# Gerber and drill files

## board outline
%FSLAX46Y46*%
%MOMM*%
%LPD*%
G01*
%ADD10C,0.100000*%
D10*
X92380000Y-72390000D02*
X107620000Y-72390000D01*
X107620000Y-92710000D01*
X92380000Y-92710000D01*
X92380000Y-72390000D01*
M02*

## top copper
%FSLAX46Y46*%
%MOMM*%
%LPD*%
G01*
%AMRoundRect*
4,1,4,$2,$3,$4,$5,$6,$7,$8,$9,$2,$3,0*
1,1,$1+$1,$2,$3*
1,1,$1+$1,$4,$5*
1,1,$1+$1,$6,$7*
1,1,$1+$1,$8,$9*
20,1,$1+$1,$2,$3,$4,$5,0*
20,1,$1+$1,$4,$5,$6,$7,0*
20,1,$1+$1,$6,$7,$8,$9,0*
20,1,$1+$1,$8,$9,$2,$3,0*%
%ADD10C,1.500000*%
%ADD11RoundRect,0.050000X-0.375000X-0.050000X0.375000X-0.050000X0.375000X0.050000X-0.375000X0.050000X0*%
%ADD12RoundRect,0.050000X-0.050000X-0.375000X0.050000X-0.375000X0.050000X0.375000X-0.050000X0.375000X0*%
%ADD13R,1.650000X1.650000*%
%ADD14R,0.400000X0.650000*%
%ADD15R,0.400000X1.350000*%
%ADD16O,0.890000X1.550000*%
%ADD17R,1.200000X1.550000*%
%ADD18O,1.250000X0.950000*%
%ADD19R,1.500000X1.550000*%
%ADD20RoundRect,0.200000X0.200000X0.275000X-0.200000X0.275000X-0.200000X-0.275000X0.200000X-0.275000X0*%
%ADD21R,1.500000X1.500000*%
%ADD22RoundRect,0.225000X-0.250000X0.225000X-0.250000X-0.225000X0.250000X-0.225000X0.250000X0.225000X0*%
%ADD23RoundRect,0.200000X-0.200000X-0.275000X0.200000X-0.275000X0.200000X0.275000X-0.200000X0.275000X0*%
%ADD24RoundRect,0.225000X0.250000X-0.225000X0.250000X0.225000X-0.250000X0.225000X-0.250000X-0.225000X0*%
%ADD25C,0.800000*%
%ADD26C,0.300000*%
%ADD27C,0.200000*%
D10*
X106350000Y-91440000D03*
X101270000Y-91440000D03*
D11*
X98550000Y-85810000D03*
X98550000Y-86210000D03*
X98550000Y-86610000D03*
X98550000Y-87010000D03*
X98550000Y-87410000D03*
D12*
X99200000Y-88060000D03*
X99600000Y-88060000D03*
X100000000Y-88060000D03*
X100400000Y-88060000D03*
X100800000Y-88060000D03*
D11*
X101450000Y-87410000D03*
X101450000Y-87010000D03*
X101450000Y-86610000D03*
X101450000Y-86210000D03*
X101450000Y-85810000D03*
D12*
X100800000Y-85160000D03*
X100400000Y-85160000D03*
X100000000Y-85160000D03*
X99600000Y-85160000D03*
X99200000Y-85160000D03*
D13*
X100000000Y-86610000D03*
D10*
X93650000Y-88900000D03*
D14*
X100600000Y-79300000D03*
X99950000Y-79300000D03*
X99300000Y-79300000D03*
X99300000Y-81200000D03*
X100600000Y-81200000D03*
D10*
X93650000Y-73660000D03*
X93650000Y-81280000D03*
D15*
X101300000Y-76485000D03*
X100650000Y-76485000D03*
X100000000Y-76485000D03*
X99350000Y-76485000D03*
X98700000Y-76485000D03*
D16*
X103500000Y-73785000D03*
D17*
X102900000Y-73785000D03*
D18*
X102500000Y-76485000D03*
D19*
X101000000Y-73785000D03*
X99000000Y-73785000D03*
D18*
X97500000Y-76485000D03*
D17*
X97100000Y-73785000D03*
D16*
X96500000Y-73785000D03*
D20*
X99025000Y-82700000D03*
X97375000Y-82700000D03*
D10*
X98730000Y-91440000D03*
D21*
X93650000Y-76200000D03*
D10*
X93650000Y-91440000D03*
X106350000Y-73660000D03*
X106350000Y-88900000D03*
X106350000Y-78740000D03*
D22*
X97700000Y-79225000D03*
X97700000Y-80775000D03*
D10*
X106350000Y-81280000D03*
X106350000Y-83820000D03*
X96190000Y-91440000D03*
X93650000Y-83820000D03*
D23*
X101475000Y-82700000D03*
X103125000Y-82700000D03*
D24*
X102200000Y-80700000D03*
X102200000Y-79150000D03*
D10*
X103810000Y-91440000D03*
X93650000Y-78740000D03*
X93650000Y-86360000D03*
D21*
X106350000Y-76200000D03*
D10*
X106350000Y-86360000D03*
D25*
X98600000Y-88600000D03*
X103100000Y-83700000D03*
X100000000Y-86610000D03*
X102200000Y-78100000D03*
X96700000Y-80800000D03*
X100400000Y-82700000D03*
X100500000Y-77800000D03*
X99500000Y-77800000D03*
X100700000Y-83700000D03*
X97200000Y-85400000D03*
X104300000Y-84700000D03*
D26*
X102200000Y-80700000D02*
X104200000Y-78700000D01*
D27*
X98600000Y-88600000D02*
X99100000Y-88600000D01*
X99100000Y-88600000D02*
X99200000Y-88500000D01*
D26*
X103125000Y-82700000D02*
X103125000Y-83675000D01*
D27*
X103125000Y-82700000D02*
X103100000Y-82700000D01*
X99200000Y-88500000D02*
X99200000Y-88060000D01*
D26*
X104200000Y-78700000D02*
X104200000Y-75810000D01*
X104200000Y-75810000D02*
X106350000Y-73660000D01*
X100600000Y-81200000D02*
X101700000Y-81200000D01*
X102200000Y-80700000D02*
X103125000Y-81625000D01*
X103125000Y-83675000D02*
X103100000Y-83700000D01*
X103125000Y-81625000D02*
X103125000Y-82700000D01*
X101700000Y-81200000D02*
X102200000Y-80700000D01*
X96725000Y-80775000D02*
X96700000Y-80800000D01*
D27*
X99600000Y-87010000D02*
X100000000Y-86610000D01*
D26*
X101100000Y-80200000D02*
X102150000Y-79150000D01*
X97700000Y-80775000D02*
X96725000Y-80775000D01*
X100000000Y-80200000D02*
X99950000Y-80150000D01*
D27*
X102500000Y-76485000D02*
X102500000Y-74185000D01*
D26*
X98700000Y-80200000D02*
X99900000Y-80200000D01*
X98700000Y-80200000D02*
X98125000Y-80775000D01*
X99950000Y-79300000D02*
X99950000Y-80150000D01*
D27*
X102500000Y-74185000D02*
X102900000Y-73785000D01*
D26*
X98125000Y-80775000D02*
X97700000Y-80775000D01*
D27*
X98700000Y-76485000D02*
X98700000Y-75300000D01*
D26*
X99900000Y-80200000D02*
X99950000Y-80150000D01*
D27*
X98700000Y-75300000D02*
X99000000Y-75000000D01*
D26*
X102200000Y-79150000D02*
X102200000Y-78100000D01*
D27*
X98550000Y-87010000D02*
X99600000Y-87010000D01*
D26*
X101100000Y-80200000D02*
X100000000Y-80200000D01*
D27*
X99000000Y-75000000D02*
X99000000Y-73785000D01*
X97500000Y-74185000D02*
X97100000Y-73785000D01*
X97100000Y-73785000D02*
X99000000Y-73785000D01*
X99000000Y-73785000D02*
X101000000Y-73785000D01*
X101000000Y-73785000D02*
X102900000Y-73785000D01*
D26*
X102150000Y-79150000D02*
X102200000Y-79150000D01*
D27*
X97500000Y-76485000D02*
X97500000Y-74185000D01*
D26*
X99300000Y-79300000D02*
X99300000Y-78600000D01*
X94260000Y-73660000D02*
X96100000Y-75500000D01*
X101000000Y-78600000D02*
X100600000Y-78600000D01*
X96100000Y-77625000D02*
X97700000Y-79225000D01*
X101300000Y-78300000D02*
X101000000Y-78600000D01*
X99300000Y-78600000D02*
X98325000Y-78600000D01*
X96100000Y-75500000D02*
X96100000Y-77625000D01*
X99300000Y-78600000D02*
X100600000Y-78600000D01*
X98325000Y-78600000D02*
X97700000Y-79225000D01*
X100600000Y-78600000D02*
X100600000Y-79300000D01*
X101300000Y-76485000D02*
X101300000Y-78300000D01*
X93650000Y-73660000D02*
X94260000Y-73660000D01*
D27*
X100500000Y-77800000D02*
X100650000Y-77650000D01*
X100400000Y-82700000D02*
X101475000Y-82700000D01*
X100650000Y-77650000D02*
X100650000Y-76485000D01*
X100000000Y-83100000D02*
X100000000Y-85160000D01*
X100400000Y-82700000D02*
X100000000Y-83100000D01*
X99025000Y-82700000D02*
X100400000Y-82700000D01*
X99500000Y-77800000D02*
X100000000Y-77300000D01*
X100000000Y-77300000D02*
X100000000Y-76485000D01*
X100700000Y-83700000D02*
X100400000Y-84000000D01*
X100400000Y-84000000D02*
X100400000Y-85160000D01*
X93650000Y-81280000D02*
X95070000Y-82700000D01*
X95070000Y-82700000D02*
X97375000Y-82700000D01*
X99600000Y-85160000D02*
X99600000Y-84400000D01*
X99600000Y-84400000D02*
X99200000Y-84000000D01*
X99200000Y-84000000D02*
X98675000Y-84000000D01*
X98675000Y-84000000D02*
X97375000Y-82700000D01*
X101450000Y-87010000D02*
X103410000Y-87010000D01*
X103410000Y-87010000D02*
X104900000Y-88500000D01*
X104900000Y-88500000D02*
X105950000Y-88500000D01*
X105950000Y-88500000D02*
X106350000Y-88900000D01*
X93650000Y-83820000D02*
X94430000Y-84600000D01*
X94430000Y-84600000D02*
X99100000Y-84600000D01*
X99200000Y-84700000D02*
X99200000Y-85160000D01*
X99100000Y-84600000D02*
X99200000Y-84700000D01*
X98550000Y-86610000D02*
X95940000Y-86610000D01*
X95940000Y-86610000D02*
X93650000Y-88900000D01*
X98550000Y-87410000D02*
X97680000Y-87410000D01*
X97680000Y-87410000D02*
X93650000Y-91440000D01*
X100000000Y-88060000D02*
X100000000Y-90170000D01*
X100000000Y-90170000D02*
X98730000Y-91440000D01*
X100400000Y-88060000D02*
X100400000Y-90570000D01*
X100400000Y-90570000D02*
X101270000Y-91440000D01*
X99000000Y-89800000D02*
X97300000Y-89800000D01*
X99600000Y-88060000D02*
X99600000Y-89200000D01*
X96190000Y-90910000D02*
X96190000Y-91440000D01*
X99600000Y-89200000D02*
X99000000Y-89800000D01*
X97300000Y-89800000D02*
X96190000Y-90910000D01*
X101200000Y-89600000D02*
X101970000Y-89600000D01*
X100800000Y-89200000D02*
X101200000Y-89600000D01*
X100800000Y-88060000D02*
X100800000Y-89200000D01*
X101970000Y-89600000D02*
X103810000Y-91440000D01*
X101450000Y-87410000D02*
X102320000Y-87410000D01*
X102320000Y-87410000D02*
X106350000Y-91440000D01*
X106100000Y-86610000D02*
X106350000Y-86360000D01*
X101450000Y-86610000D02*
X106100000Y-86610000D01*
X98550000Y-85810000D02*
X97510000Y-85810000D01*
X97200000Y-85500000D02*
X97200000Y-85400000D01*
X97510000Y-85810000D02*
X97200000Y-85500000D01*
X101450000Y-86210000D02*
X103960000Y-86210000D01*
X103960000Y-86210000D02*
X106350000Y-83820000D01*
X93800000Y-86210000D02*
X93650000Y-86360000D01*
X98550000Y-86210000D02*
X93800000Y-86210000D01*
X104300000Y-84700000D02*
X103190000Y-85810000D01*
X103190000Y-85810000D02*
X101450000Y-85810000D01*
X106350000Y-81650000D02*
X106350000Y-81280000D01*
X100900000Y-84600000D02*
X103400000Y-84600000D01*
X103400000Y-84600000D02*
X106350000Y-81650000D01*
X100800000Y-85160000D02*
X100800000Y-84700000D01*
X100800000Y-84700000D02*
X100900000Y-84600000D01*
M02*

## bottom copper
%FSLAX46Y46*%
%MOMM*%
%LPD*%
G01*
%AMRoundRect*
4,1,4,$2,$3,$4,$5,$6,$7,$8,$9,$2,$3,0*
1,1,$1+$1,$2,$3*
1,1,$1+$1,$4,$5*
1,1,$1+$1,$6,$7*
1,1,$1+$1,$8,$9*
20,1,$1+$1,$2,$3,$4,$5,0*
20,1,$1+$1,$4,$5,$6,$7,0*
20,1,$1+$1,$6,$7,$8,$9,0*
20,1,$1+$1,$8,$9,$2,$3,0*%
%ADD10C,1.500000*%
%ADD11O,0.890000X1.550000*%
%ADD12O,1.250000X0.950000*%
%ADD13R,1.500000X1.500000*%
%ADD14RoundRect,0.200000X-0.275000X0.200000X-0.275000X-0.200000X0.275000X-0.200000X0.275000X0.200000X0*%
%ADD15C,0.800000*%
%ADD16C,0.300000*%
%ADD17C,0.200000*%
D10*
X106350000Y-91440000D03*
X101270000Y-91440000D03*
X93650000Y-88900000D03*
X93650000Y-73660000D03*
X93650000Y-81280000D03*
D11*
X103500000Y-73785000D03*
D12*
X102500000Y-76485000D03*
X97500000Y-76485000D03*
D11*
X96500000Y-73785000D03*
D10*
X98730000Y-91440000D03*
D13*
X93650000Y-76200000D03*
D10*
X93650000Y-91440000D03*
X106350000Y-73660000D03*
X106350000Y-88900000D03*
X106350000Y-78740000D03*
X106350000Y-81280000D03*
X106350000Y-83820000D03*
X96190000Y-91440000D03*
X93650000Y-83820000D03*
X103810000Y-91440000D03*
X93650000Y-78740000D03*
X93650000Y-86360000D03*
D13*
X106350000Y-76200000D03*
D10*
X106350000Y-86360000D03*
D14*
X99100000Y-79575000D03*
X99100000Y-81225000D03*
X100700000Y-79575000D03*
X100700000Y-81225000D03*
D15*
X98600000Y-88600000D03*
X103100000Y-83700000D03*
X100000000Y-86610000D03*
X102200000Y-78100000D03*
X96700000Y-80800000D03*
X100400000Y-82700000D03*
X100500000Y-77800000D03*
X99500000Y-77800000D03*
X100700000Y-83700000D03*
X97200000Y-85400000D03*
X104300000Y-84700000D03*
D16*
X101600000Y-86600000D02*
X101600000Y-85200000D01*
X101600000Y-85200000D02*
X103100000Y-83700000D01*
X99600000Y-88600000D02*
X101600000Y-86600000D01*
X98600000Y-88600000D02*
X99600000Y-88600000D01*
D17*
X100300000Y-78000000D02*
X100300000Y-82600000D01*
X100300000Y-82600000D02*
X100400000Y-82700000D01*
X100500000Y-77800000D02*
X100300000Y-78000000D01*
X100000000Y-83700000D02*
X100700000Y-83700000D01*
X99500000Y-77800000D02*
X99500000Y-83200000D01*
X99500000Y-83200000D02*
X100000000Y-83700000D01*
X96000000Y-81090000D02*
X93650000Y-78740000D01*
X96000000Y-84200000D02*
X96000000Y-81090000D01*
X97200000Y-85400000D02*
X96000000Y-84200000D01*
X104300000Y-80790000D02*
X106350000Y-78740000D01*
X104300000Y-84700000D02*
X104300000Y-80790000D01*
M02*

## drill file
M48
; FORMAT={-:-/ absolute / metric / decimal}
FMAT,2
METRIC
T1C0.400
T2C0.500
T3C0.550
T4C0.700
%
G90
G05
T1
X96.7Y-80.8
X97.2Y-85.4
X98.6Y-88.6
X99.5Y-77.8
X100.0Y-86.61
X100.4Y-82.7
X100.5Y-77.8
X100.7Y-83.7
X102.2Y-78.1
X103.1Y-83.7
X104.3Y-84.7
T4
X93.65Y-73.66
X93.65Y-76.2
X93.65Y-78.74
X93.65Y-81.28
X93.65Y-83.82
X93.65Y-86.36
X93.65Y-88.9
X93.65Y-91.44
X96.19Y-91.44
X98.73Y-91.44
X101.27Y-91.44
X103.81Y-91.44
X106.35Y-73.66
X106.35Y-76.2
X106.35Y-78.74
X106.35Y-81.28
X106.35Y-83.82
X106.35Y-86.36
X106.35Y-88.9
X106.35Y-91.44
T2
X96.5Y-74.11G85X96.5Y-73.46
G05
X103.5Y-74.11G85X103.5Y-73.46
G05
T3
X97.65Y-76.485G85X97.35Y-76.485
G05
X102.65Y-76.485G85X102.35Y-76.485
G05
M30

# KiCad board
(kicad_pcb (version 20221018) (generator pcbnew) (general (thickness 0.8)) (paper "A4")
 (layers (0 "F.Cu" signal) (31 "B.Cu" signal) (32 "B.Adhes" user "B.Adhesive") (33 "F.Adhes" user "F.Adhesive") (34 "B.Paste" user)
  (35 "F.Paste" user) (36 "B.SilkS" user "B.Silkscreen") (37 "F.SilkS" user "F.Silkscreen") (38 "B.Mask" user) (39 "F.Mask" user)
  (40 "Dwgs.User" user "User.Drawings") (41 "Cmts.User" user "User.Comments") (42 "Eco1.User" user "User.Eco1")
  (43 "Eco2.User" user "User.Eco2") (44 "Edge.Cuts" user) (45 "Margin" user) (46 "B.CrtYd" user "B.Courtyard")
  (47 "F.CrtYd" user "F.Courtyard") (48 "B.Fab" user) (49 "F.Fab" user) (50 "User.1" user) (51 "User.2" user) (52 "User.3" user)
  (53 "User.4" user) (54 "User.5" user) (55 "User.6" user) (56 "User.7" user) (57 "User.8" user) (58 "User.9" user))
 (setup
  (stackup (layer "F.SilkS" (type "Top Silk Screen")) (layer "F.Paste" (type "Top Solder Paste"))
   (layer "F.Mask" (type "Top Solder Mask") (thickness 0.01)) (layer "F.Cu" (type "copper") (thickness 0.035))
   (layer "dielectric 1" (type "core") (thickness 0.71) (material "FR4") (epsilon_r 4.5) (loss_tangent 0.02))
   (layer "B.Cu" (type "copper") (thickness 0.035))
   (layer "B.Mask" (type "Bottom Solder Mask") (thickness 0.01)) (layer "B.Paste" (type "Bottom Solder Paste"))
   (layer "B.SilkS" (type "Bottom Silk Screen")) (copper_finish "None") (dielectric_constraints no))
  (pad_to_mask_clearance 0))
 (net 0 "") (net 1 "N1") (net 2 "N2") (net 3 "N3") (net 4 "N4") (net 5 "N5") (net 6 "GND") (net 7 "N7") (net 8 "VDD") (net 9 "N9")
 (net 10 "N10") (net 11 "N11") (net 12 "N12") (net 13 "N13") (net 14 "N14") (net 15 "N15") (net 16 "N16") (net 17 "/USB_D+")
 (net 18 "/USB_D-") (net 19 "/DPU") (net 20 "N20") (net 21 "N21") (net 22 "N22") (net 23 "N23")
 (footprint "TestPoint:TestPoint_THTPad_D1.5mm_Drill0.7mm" (layer "F.Cu") (at 106.35 91.44 -90)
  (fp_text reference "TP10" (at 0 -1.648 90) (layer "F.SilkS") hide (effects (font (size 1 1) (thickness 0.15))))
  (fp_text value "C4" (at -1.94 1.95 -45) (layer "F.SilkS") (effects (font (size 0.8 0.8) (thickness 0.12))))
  (pad "1" thru_hole circle (at 0 0 270) (size 1.5 1.5) (drill 0.7) (layers "*.Cu" "*.Mask") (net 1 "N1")))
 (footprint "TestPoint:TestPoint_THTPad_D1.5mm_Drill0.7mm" (layer "F.Cu") (at 101.27 91.44 -90)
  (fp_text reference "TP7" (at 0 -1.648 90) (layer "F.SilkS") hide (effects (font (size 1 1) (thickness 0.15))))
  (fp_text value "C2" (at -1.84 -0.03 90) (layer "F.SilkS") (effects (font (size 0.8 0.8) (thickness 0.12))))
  (pad "1" thru_hole circle (at 0 0 270) (size 1.5 1.5) (drill 0.7) (layers "*.Cu" "*.Mask") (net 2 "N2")))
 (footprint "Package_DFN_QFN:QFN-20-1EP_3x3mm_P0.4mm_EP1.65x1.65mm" (layer "F.Cu") (at 100 86.61)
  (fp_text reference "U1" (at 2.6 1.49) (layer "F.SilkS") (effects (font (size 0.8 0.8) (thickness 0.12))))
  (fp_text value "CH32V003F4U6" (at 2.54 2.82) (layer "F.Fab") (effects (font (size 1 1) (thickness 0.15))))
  (pad "" smd roundrect (at -0.41 -0.41) (size 0.67 0.67) (layers "F.Paste") (roundrect_rratio 0.25))
  (pad "" smd roundrect (at -0.41 0.41) (size 0.67 0.67) (layers "F.Paste") (roundrect_rratio 0.25))
  (pad "" smd roundrect (at 0.41 -0.41) (size 0.67 0.67) (layers "F.Paste") (roundrect_rratio 0.25))
  (pad "" smd roundrect (at 0.41 0.41) (size 0.67 0.67) (layers "F.Paste") (roundrect_rratio 0.25))
  (pad "1" smd roundrect (at -1.45 -0.8) (size 0.85 0.2) (layers "F.Cu" "F.Paste" "F.Mask") (roundrect_rratio 0.25) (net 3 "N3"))
  (pad "2" smd roundrect (at -1.45 -0.4) (size 0.85 0.2) (layers "F.Cu" "F.Paste" "F.Mask") (roundrect_rratio 0.25) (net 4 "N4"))
  (pad "3" smd roundrect (at -1.45 0) (size 0.85 0.2) (layers "F.Cu" "F.Paste" "F.Mask") (roundrect_rratio 0.25) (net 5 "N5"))
  (pad "4" smd roundrect (at -1.45 0.4) (size 0.85 0.2) (layers "F.Cu" "F.Paste" "F.Mask") (roundrect_rratio 0.25) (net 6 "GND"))
  (pad "5" smd roundrect (at -1.45 0.8) (size 0.85 0.2) (layers "F.Cu" "F.Paste" "F.Mask") (roundrect_rratio 0.25) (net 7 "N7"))
  (pad "6" smd roundrect (at -0.8 1.45) (size 0.2 0.85) (layers "F.Cu" "F.Paste" "F.Mask") (roundrect_rratio 0.25) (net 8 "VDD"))
  (pad "7" smd roundrect (at -0.4 1.45) (size 0.2 0.85) (layers "F.Cu" "F.Paste" "F.Mask") (roundrect_rratio 0.25) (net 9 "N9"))
  (pad "8" smd roundrect (at 0 1.45) (size 0.2 0.85) (layers "F.Cu" "F.Paste" "F.Mask") (roundrect_rratio 0.25) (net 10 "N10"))
  (pad "9" smd roundrect (at 0.4 1.45) (size 0.2 0.85) (layers "F.Cu" "F.Paste" "F.Mask") (roundrect_rratio 0.25) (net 2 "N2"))
  (pad "10" smd roundrect (at 0.8 1.45) (size 0.2 0.85) (layers "F.Cu" "F.Paste" "F.Mask") (roundrect_rratio 0.25) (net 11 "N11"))
  (pad "11" smd roundrect (at 1.45 0.8) (size 0.85 0.2) (layers "F.Cu" "F.Paste" "F.Mask") (roundrect_rratio 0.25) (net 1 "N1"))
  (pad "12" smd roundrect (at 1.45 0.4) (size 0.85 0.2) (layers "F.Cu" "F.Paste" "F.Mask") (roundrect_rratio 0.25) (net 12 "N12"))
  (pad "13" smd roundrect (at 1.45 0) (size 0.85 0.2) (layers "F.Cu" "F.Paste" "F.Mask") (roundrect_rratio 0.25) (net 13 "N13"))
  (pad "14" smd roundrect (at 1.45 -0.4) (size 0.85 0.2) (layers "F.Cu" "F.Paste" "F.Mask") (roundrect_rratio 0.25) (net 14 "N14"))
  (pad "15" smd roundrect (at 1.45 -0.8) (size 0.85 0.2) (layers "F.Cu" "F.Paste" "F.Mask") (roundrect_rratio 0.25) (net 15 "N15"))
  (pad "16" smd roundrect (at 0.8 -1.45) (size 0.2 0.85) (layers "F.Cu" "F.Paste" "F.Mask") (roundrect_rratio 0.25) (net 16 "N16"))
  (pad "17" smd roundrect (at 0.4 -1.45) (size 0.2 0.85) (layers "F.Cu" "F.Paste" "F.Mask") (roundrect_rratio 0.25) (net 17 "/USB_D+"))
  (pad "18" smd roundrect (at 0 -1.45) (size 0.2 0.85) (layers "F.Cu" "F.Paste" "F.Mask") (roundrect_rratio 0.25) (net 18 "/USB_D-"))
  (pad "19" smd roundrect (at -0.4 -1.45) (size 0.2 0.85) (layers "F.Cu" "F.Paste" "F.Mask") (roundrect_rratio 0.25) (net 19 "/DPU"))
  (pad "20" smd roundrect (at -0.8 -1.45) (size 0.2 0.85) (layers "F.Cu" "F.Paste" "F.Mask") (roundrect_rratio 0.25) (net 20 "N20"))
  (pad "21" smd rect (at 0 0) (size 1.65 1.65) (layers "F.Cu" "F.Mask") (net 6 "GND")))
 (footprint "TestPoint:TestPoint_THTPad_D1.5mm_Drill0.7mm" (layer "F.Cu") (at 93.65 88.9 180)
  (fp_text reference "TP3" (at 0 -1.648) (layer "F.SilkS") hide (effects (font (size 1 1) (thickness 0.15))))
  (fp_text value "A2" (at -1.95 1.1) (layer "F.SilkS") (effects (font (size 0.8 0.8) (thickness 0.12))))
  (pad "1" thru_hole circle (at 0 0 180) (size 1.5 1.5) (drill 0.7) (layers "*.Cu" "*.Mask") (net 5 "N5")))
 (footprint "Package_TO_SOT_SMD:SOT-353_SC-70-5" (layer "F.Cu") (at 99.95 80.25 -90)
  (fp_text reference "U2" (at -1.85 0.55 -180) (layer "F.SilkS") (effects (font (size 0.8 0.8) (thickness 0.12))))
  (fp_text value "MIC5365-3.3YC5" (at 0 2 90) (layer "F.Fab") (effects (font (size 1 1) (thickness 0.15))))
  (pad "1" smd rect (at -0.95 -0.65 270) (size 0.65 0.4) (layers "F.Cu" "F.Paste" "F.Mask") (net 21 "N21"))
  (pad "2" smd rect (at -0.95 0 270) (size 0.65 0.4) (layers "F.Cu" "F.Paste" "F.Mask") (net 6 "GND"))
  (pad "3" smd rect (at -0.95 0.65 270) (size 0.65 0.4) (layers "F.Cu" "F.Paste" "F.Mask") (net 21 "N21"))
  (pad "4" smd rect (at 0.95 0.65 270) (size 0.65 0.4) (layers "F.Cu" "F.Paste" "F.Mask") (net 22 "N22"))
  (pad "5" smd rect (at 0.95 -0.65 270) (size 0.65 0.4) (layers "F.Cu" "F.Paste" "F.Mask") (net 8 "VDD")))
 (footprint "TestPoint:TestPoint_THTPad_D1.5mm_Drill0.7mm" (layer "F.Cu") (at 93.65 73.66 -90)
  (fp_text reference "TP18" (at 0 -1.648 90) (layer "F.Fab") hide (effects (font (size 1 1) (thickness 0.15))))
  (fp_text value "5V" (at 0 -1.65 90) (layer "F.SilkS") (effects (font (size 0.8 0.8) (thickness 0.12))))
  (pad "1" thru_hole circle (at 0 0 270) (size 1.5 1.5) (drill 0.7) (layers "*.Cu" "*.Mask") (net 21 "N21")))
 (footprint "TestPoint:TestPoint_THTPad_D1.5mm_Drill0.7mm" (layer "F.Cu") (at 93.65 81.28)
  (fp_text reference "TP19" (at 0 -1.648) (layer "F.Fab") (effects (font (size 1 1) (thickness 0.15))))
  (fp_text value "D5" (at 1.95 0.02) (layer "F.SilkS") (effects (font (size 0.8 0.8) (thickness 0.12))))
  (pad "1" thru_hole circle (at 0 0) (size 1.5 1.5) (drill 0.7) (layers "*.Cu" "*.Mask") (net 19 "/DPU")))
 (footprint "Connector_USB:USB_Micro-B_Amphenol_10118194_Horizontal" (layer "F.Cu") (at 100 75.085 180)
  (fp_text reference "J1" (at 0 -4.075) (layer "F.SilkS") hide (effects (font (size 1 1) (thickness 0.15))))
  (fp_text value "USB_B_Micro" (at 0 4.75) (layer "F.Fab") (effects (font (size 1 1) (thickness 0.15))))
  (pad "" smd oval (at -3.5 1.3 180) (size 0.89 1.55) (layers "F.Paste"))
  (pad "" smd oval (at -2.5 -1.4 180) (size 1.25 0.95) (layers "F.Paste"))
  (pad "" smd oval (at 2.5 -1.4 180) (size 1.25 0.95) (layers "F.Paste"))
  (pad "" smd oval (at 3.5 1.3 180) (size 0.89 1.55) (layers "F.Paste"))
  (pad "1" smd rect (at -1.3 -1.4 180) (size 0.4 1.35) (layers "F.Cu" "F.Paste" "F.Mask") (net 21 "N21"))
  (pad "2" smd rect (at -0.65 -1.4 180) (size 0.4 1.35) (layers "F.Cu" "F.Paste" "F.Mask") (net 18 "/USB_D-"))
  (pad "3" smd rect (at 0 -1.4 180) (size 0.4 1.35) (layers "F.Cu" "F.Paste" "F.Mask") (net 17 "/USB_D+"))
  (pad "4" smd rect (at 0.65 -1.4 180) (size 0.4 1.35) (layers "F.Cu" "F.Paste" "F.Mask") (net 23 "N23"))
  (pad "5" smd rect (at 1.3 -1.4 180) (size 0.4 1.35) (layers "F.Cu" "F.Paste" "F.Mask") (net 6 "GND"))
  (pad "6" thru_hole oval (at -3.5 1.3 180) (size 0.89 1.55) (drill oval 0.5 1.15) (layers "*.Cu" "*.Mask") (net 6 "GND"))
  (pad "6" smd rect (at -2.9 1.3 180) (size 1.2 1.55) (layers "F.Cu" "F.Paste" "F.Mask") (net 6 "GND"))
  (pad "6" thru_hole oval (at -2.5 -1.4 180) (size 1.25 0.95) (drill oval 0.85 0.55) (layers "*.Cu" "*.Mask") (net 6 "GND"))
  (pad "6" smd rect (at -1 1.3 180) (size 1.5 1.55) (layers "F.Cu" "F.Paste" "F.Mask") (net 6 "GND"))
  (pad "6" smd rect (at 1 1.3 180) (size 1.5 1.55) (layers "F.Cu" "F.Paste" "F.Mask") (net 6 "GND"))
  (pad "6" thru_hole oval (at 2.5 -1.4 180) (size 1.25 0.95) (drill oval 0.85 0.55) (layers "*.Cu" "*.Mask") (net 6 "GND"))
  (pad "6" smd rect (at 2.9 1.3 180) (size 1.2 1.55) (layers "F.Cu" "F.Paste" "F.Mask") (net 6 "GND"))
  (pad "6" thru_hole oval (at 3.5 1.3 180) (size 0.89 1.55) (drill oval 0.5 1.15) (layers "*.Cu" "*.Mask") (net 6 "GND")))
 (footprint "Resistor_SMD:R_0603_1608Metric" (layer "F.Cu") (at 98.2 82.7 180)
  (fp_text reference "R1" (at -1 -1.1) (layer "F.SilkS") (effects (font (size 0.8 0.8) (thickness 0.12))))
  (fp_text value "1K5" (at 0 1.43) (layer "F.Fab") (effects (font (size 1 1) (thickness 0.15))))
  (pad "1" smd roundrect (at -0.825 0 180) (size 0.8 0.95) (layers "F.Cu" "F.Paste" "F.Mask") (roundrect_rratio 0.25) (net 18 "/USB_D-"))
  (pad "2" smd roundrect (at 0.825 0 180) (size 0.8 0.95) (layers "F.Cu" "F.Paste" "F.Mask") (roundrect_rratio 0.25) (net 19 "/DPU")))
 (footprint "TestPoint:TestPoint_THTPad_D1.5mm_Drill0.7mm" (layer "F.Cu") (at 98.73 91.44 -90)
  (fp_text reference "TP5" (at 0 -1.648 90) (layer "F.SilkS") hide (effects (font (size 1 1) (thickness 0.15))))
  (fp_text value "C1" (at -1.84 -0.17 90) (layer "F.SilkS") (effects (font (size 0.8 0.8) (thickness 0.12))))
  (pad "1" thru_hole circle (at 0 0 270) (size 1.5 1.5) (drill 0.7) (layers "*.Cu" "*.Mask") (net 10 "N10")))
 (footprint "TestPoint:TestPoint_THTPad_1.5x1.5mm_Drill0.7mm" (layer "F.Cu") (at 93.65 76.2 180)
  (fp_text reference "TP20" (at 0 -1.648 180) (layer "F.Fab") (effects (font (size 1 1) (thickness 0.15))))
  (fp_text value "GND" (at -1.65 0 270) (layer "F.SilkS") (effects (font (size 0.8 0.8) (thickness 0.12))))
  (pad "1" thru_hole rect (at 0 0 180) (size 1.5 1.5) (drill 0.7) (layers "*.Cu" "*.Mask") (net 6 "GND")))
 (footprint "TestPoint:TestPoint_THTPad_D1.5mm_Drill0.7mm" (layer "F.Cu") (at 93.65 91.44 180)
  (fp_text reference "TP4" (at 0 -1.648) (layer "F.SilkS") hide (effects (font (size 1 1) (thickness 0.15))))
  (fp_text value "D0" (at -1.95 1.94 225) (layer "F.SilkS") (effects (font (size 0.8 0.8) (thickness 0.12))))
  (pad "1" thru_hole circle (at 0 0 180) (size 1.5 1.5) (drill 0.7) (layers "*.Cu" "*.Mask") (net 7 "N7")))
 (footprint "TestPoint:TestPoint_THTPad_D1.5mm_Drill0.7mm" (layer "F.Cu") (at 106.35 73.66)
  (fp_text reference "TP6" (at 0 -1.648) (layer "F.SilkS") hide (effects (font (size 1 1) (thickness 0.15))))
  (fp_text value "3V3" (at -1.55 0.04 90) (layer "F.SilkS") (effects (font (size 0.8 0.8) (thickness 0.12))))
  (pad "1" thru_hole circle (at 0 0) (size 1.5 1.5) (drill 0.7) (layers "*.Cu" "*.Mask") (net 8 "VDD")))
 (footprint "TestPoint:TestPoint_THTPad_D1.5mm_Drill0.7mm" (layer "F.Cu") (at 106.35 88.9)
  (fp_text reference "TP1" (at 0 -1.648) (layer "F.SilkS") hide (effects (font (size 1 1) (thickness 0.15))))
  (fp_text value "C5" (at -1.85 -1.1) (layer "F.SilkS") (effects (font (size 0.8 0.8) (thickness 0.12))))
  (pad "1" thru_hole circle (at 0 0) (size 1.5 1.5) (drill 0.7) (layers "*.Cu" "*.Mask") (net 12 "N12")))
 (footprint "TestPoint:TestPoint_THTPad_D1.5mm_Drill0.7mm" (layer "F.Cu") (at 106.35 78.74)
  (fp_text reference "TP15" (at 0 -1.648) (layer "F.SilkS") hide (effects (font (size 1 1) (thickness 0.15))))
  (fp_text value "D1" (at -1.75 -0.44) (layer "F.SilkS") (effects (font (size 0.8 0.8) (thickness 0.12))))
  (pad "1" thru_hole circle (at 0 0) (size 1.5 1.5) (drill 0.7) (layers "*.Cu" "*.Mask") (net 15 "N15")))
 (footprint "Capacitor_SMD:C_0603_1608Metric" (layer "F.Cu") (at 97.7 80 -90)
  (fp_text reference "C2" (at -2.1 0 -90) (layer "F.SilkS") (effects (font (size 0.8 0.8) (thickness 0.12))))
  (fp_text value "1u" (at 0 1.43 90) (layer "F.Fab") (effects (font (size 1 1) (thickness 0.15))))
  (pad "1" smd roundrect (at -0.775 0 270) (size 0.9 0.95) (layers "F.Cu" "F.Paste" "F.Mask") (roundrect_rratio 0.25) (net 21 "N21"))
  (pad "2" smd roundrect (at 0.775 0 270) (size 0.9 0.95) (layers "F.Cu" "F.Paste" "F.Mask") (roundrect_rratio 0.25) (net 6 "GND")))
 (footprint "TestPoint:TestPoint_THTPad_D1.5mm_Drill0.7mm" (layer "F.Cu") (at 106.35 81.28)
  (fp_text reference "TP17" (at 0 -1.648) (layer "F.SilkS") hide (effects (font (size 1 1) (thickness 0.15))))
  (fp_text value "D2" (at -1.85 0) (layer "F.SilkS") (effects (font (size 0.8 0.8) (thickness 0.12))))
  (pad "1" thru_hole circle (at 0 0) (size 1.5 1.5) (drill 0.7) (layers "*.Cu" "*.Mask") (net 16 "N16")))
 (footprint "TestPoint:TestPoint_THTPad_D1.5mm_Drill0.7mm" (layer "F.Cu") (at 106.35 83.82)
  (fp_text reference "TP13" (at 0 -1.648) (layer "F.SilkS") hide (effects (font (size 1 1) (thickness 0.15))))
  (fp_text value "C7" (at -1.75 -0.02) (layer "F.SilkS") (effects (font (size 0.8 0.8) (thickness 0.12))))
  (pad "1" thru_hole circle (at 0 0) (size 1.5 1.5) (drill 0.7) (layers "*.Cu" "*.Mask") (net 14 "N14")))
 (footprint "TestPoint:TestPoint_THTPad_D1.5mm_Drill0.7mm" (layer "F.Cu") (at 96.19 91.44 -90)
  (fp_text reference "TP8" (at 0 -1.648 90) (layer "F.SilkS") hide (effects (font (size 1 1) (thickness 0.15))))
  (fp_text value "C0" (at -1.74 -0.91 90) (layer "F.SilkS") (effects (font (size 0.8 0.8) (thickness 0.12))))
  (pad "1" thru_hole circle (at 0 0 270) (size 1.5 1.5) (drill 0.7) (layers "*.Cu" "*.Mask") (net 9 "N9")))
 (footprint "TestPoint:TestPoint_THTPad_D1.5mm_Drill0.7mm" (layer "F.Cu") (at 93.65 83.82 180)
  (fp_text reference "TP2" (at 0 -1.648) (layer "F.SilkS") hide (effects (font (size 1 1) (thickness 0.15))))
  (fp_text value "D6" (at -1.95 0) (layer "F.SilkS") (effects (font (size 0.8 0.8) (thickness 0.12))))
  (pad "1" thru_hole circle (at 0 0 180) (size 1.5 1.5) (drill 0.7) (layers "*.Cu" "*.Mask") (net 20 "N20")))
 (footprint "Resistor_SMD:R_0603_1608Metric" (layer "F.Cu") (at 102.3 82.7)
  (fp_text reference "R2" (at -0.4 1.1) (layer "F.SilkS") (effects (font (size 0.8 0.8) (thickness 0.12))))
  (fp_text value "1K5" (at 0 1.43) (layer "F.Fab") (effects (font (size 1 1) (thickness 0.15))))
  (pad "1" smd roundrect (at -0.825 0) (size 0.8 0.95) (layers "F.Cu" "F.Paste" "F.Mask") (roundrect_rratio 0.25) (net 18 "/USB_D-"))
  (pad "2" smd roundrect (at 0.825 0) (size 0.8 0.95) (layers "F.Cu" "F.Paste" "F.Mask") (roundrect_rratio 0.25) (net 8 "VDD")))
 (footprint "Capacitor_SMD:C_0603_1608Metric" (layer "F.Cu") (at 102.2 79.925 90)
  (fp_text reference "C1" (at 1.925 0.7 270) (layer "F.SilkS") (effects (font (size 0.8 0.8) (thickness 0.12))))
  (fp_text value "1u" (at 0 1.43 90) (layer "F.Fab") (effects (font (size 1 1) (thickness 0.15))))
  (pad "1" smd roundrect (at -0.775 0 90) (size 0.9 0.95) (layers "F.Cu" "F.Paste" "F.Mask") (roundrect_rratio 0.25) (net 8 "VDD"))
  (pad "2" smd roundrect (at 0.775 0 90) (size 0.9 0.95) (layers "F.Cu" "F.Paste" "F.Mask") (roundrect_rratio 0.25) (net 6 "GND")))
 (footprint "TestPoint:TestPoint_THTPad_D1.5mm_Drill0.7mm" (layer "F.Cu") (at 103.81 91.44 -90)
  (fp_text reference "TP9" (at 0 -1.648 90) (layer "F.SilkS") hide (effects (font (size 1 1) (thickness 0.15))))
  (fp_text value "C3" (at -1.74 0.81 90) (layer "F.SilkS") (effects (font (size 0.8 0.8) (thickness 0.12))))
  (pad "1" thru_hole circle (at 0 0 270) (size 1.5 1.5) (drill 0.7) (layers "*.Cu" "*.Mask") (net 11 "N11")))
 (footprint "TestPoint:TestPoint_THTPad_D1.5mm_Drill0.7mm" (layer "F.Cu") (at 93.65 78.74 180)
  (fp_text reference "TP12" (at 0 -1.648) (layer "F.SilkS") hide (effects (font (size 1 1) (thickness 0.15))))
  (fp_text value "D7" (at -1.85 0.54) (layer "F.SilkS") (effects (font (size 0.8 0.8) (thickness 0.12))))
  (pad "1" thru_hole circle (at 0 0 180) (size 1.5 1.5) (drill 0.7) (layers "*.Cu" "*.Mask") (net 3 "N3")))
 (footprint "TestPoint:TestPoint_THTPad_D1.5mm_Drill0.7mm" (layer "F.Cu") (at 93.65 86.36 180)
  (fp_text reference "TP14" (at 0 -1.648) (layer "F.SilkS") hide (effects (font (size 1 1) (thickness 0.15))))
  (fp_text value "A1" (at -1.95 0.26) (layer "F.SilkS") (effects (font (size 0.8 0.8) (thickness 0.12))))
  (pad "1" thru_hole circle (at 0 0 180) (size 1.5 1.5) (drill 0.7) (layers "*.Cu" "*.Mask") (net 4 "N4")))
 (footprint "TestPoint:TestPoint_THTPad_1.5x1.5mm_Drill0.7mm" (layer "F.Cu") (at 106.35 76.2)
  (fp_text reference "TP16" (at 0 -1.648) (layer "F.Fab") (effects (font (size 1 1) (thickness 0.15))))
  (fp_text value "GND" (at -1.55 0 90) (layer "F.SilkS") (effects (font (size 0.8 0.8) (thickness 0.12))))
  (pad "1" thru_hole rect (at 0 0) (size 1.5 1.5) (drill 0.7) (layers "*.Cu" "*.Mask") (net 6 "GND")))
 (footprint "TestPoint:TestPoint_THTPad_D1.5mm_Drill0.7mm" (layer "F.Cu") (at 106.35 86.36)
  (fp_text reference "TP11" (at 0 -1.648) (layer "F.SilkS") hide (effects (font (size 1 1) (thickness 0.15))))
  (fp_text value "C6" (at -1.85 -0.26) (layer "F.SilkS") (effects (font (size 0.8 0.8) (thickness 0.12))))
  (pad "1" thru_hole circle (at 0 0) (size 1.5 1.5) (drill 0.7) (layers "*.Cu" "*.Mask") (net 13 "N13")))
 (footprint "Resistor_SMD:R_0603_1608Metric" (layer "B.Cu") (at 99.1 80.4 -90)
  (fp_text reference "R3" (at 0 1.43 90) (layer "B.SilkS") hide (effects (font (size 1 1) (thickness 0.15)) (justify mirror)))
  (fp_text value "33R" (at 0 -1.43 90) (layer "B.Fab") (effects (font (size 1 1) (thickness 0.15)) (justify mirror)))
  (pad "1" smd roundrect (at -0.825 0 270) (size 0.8 0.95) (layers "B.Cu" "B.Paste" "B.Mask") (roundrect_rratio 0.25) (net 18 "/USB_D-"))
  (pad "2" smd roundrect (at 0.825 0 270) (size 0.8 0.95) (layers "B.Cu" "B.Paste" "B.Mask") (roundrect_rratio 0.25) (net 18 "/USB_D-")))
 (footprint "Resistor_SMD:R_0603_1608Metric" (layer "B.Cu") (at 100.7 80.4 -90)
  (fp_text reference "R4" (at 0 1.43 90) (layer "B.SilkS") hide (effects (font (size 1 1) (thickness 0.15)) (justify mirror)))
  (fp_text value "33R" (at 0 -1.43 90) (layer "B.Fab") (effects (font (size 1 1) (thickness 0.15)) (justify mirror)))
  (pad "1" smd roundrect (at -0.825 0 270) (size 0.8 0.95) (layers "B.Cu" "B.Paste" "B.Mask") (roundrect_rratio 0.25) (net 17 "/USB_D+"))
  (pad "2" smd roundrect (at 0.825 0 270) (size 0.8 0.95) (layers "B.Cu" "B.Paste" "B.Mask") (roundrect_rratio 0.25) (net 17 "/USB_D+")))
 (gr_rect (start 92.38 72.39) (end 107.62 92.71) (stroke (width 0.1) (type default)) (fill none) (layer "Edge.Cuts"))
 (segment (start 102.2 80.7) (end 104.2 78.7) (width 0.3) (layer "F.Cu") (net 8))
 (segment (start 98.6 88.6) (end 99.1 88.6) (width 0.2) (layer "F.Cu") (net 8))
 (segment (start 99.1 88.6) (end 99.2 88.5) (width 0.2) (layer "F.Cu") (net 8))
 (segment (start 103.125 82.7) (end 103.125 83.675) (width 0.3) (layer "F.Cu") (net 8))
 (segment (start 103.125 82.7) (end 103.1 82.7) (width 0.2) (layer "F.Cu") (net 8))
 (segment (start 99.2 88.5) (end 99.2 88.06) (width 0.2) (layer "F.Cu") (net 8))
 (segment (start 104.2 78.7) (end 104.2 75.81) (width 0.3) (layer "F.Cu") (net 8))
 (segment (start 104.2 75.81) (end 106.35 73.66) (width 0.3) (layer "F.Cu") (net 8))
 (segment (start 100.6 81.2) (end 101.7 81.2) (width 0.3) (layer "F.Cu") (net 8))
 (segment (start 102.2 80.7) (end 103.125 81.625) (width 0.3) (layer "F.Cu") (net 8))
 (segment (start 103.125 83.675) (end 103.1 83.7) (width 0.3) (layer "F.Cu") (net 8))
 (segment (start 103.125 81.625) (end 103.125 82.7) (width 0.3) (layer "F.Cu") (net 8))
 (segment (start 101.7 81.2) (end 102.2 80.7) (width 0.3) (layer "F.Cu") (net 8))
 (via (at 98.6 88.6) (size 0.8) (drill 0.4) (layers "F.Cu" "B.Cu") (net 8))
 (via (at 103.1 83.7) (size 0.8) (drill 0.4) (layers "F.Cu" "B.Cu") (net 8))
 (segment (start 101.6 86.6) (end 101.6 85.2) (width 0.3) (layer "B.Cu") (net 8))
 (segment (start 101.6 85.2) (end 103.1 83.7) (width 0.3) (layer "B.Cu") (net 8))
 (segment (start 99.6 88.6) (end 101.6 86.6) (width 0.3) (layer "B.Cu") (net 8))
 (segment (start 98.6 88.6) (end 99.6 88.6) (width 0.3) (layer "B.Cu") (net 8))
 (segment (start 96.725 80.775) (end 96.7 80.8) (width 0.3) (layer "F.Cu") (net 6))
 (segment (start 99.6 87.01) (end 100 86.61) (width 0.2) (layer "F.Cu") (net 6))
 (segment (start 101.1 80.2) (end 102.15 79.15) (width 0.3) (layer "F.Cu") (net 6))
 (segment (start 97.7 80.775) (end 96.725 80.775) (width 0.3) (layer "F.Cu") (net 6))
 (segment (start 100 80.2) (end 99.95 80.15) (width 0.3) (layer "F.Cu") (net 6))
 (segment (start 102.5 76.485) (end 102.5 74.185) (width 0.2) (layer "F.Cu") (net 6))
 (segment (start 98.7 80.2) (end 99.9 80.2) (width 0.3) (layer "F.Cu") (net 6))
 (segment (start 98.7 80.2) (end 98.125 80.775) (width 0.3) (layer "F.Cu") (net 6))
 (segment (start 99.95 79.3) (end 99.95 80.15) (width 0.3) (layer "F.Cu") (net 6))
 (segment (start 102.5 74.185) (end 102.9 73.785) (width 0.2) (layer "F.Cu") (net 6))
 (segment (start 98.125 80.775) (end 97.7 80.775) (width 0.3) (layer "F.Cu") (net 6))
 (segment (start 98.7 76.485) (end 98.7 75.3) (width 0.2) (layer "F.Cu") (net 6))
 (segment (start 99.9 80.2) (end 99.95 80.15) (width 0.3) (layer "F.Cu") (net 6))
 (segment (start 98.7 75.3) (end 99 75) (width 0.2) (layer "F.Cu") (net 6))
 (segment (start 102.2 79.15) (end 102.2 78.1) (width 0.3) (layer "F.Cu") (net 6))
 (segment (start 98.55 87.01) (end 99.6 87.01) (width 0.2) (layer "F.Cu") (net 6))
 (segment (start 101.1 80.2) (end 100 80.2) (width 0.3) (layer "F.Cu") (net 6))
 (segment (start 99 75) (end 99 73.785) (width 0.2) (layer "F.Cu") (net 6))
 (segment (start 97.5 74.185) (end 97.1 73.785) (width 0.2) (layer "F.Cu") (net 6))
 (segment (start 97.1 73.785) (end 99 73.785) (width 0.2) (layer "F.Cu") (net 6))
 (segment (start 99 73.785) (end 101 73.785) (width 0.2) (layer "F.Cu") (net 6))
 (segment (start 101 73.785) (end 102.9 73.785) (width 0.2) (layer "F.Cu") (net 6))
 (segment (start 102.15 79.15) (end 102.2 79.15) (width 0.3) (layer "F.Cu") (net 6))
 (segment (start 97.5 76.485) (end 97.5 74.185) (width 0.2) (layer "F.Cu") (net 6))
 (via (at 100 86.61) (size 0.8) (drill 0.4) (layers "F.Cu" "B.Cu") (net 6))
 (via (at 102.2 78.1) (size 0.8) (drill 0.4) (layers "F.Cu" "B.Cu") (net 6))
 (via (at 96.7 80.8) (size 0.8) (drill 0.4) (layers "F.Cu" "B.Cu") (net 6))
 (segment (start 99.3 79.3) (end 99.3 78.6) (width 0.3) (layer "F.Cu") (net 21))
 (segment (start 94.26 73.66) (end 96.1 75.5) (width 0.3) (layer "F.Cu") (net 21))
 (segment (start 101 78.6) (end 100.6 78.6) (width 0.3) (layer "F.Cu") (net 21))
 (segment (start 96.1 77.625) (end 97.7 79.225) (width 0.3) (layer "F.Cu") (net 21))
 (segment (start 101.3 78.3) (end 101 78.6) (width 0.3) (layer "F.Cu") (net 21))
 (segment (start 99.3 78.6) (end 98.325 78.6) (width 0.3) (layer "F.Cu") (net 21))
 (segment (start 96.1 75.5) (end 96.1 77.625) (width 0.3) (layer "F.Cu") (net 21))
 (segment (start 99.3 78.6) (end 100.6 78.6) (width 0.3) (layer "F.Cu") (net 21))
 (segment (start 98.325 78.6) (end 97.7 79.225) (width 0.3) (layer "F.Cu") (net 21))
 (segment (start 100.6 78.6) (end 100.6 79.3) (width 0.3) (layer "F.Cu") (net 21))
 (segment (start 101.3 76.485) (end 101.3 78.3) (width 0.3) (layer "F.Cu") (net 21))
 (segment (start 93.65 73.66) (end 94.26 73.66) (width 0.3) (layer "F.Cu") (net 21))
 (segment (start 100.5 77.8) (end 100.65 77.65) (width 0.2) (layer "F.Cu") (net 18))
 (segment (start 100.4 82.7) (end 101.475 82.7) (width 0.2) (layer "F.Cu") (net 18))
 (segment (start 100.65 77.65) (end 100.65 76.485) (width 0.2) (layer "F.Cu") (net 18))
 (segment (start 100 83.1) (end 100 85.16) (width 0.2) (layer "F.Cu") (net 18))
 (segment (start 100.4 82.7) (end 100 83.1) (width 0.2) (layer "F.Cu") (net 18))
 (segment (start 99.025 82.7) (end 100.4 82.7) (width 0.2) (layer "F.Cu") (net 18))
 (via (at 100.4 82.7) (size 0.8) (drill 0.4) (layers "F.Cu" "B.Cu") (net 18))
 (via (at 100.5 77.8) (size 0.8) (drill 0.4) (layers "F.Cu" "B.Cu") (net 18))
 (segment (start 100.3 78) (end 100.3 82.6) (width 0.2) (layer "B.Cu") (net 18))
 (segment (start 100.3 82.6) (end 100.4 82.7) (width 0.2) (layer "B.Cu") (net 18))
 (segment (start 100.5 77.8) (end 100.3 78) (width 0.2) (layer "B.Cu") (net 18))
 (segment (start 99.5 77.8) (end 100 77.3) (width 0.2) (layer "F.Cu") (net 17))
 (segment (start 100 77.3) (end 100 76.485) (width 0.2) (layer "F.Cu") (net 17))
 (segment (start 100.7 83.7) (end 100.4 84) (width 0.2) (layer "F.Cu") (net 17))
 (segment (start 100.4 84) (end 100.4 85.16) (width 0.2) (layer "F.Cu") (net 17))
 (via (at 99.5 77.8) (size 0.8) (drill 0.4) (layers "F.Cu" "B.Cu") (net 17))
 (via (at 100.7 83.7) (size 0.8) (drill 0.4) (layers "F.Cu" "B.Cu") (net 17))
 (segment (start 100 83.7) (end 100.7 83.7) (width 0.2) (layer "B.Cu") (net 17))
 (segment (start 99.5 77.8) (end 99.5 83.2) (width 0.2) (layer "B.Cu") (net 17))
 (segment (start 99.5 83.2) (end 100 83.7) (width 0.2) (layer "B.Cu") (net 17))
 (segment (start 93.65 81.28) (end 95.07 82.7) (width 0.2) (layer "F.Cu") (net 19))
 (segment (start 95.07 82.7) (end 97.375 82.7) (width 0.2) (layer "F.Cu") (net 19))
 (segment (start 99.6 85.16) (end 99.6 84.4) (width 0.2) (layer "F.Cu") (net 19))
 (segment (start 99.6 84.4) (end 99.2 84) (width 0.2) (layer "F.Cu") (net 19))
 (segment (start 99.2 84) (end 98.675 84) (width 0.2) (layer "F.Cu") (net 19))
 (segment (start 98.675 84) (end 97.375 82.7) (width 0.2) (layer "F.Cu") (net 19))
 (segment (start 101.45 87.01) (end 103.41 87.01) (width 0.2) (layer "F.Cu") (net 12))
 (segment (start 103.41 87.01) (end 104.9 88.5) (width 0.2) (layer "F.Cu") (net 12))
 (segment (start 104.9 88.5) (end 105.95 88.5) (width 0.2) (layer "F.Cu") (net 12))
 (segment (start 105.95 88.5) (end 106.35 88.9) (width 0.2) (layer "F.Cu") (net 12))
 (segment (start 93.65 83.82) (end 94.43 84.6) (width 0.2) (layer "F.Cu") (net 20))
 (segment (start 94.43 84.6) (end 99.1 84.6) (width 0.2) (layer "F.Cu") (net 20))
 (segment (start 99.2 84.7) (end 99.2 85.16) (width 0.2) (layer "F.Cu") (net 20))
 (segment (start 99.1 84.6) (end 99.2 84.7) (width 0.2) (layer "F.Cu") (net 20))
 (segment (start 98.55 86.61) (end 95.94 86.61) (width 0.2) (layer "F.Cu") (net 5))
 (segment (start 95.94 86.61) (end 93.65 88.9) (width 0.2) (layer "F.Cu") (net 5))
 (segment (start 98.55 87.41) (end 97.68 87.41) (width 0.2) (layer "F.Cu") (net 7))
 (segment (start 97.68 87.41) (end 93.65 91.44) (width 0.2) (layer "F.Cu") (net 7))
 (segment (start 100 88.06) (end 100 90.17) (width 0.2) (layer "F.Cu") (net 10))
 (segment (start 100 90.17) (end 98.73 91.44) (width 0.2) (layer "F.Cu") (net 10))
 (segment (start 100.4 88.06) (end 100.4 90.57) (width 0.2) (layer "F.Cu") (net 2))
 (segment (start 100.4 90.57) (end 101.27 91.44) (width 0.2) (layer "F.Cu") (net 2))
 (segment (start 99 89.8) (end 97.3 89.8) (width 0.2) (layer "F.Cu") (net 9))
 (segment (start 99.6 88.06) (end 99.6 89.2) (width 0.2) (layer "F.Cu") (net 9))
 (segment (start 96.19 90.91) (end 96.19 91.44) (width 0.2) (layer "F.Cu") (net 9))
 (segment (start 99.6 89.2) (end 99 89.8) (width 0.2) (layer "F.Cu") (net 9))
 (segment (start 97.3 89.8) (end 96.19 90.91) (width 0.2) (layer "F.Cu") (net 9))
 (segment (start 101.2 89.6) (end 101.97 89.6) (width 0.2) (layer "F.Cu") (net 11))
 (segment (start 100.8 89.2) (end 101.2 89.6) (width 0.2) (layer "F.Cu") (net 11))
 (segment (start 100.8 88.06) (end 100.8 89.2) (width 0.2) (layer "F.Cu") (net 11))
 (segment (start 101.97 89.6) (end 103.81 91.44) (width 0.2) (layer "F.Cu") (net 11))
 (segment (start 101.45 87.41) (end 102.32 87.41) (width 0.2) (layer "F.Cu") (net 1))
 (segment (start 102.32 87.41) (end 106.35 91.44) (width 0.2) (layer "F.Cu") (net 1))
 (segment (start 106.1 86.61) (end 106.35 86.36) (width 0.2) (layer "F.Cu") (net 13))
 (segment (start 101.45 86.61) (end 106.1 86.61) (width 0.2) (layer "F.Cu") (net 13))
 (segment (start 98.55 85.81) (end 97.51 85.81) (width 0.2) (layer "F.Cu") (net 3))
 (segment (start 97.2 85.5) (end 97.2 85.4) (width 0.2) (layer "F.Cu") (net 3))
 (segment (start 97.51 85.81) (end 97.2 85.5) (width 0.2) (layer "F.Cu") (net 3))
 (via (at 97.2 85.4) (size 0.8) (drill 0.4) (layers "F.Cu" "B.Cu") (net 3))
 (segment (start 96 81.09) (end 93.65 78.74) (width 0.2) (layer "B.Cu") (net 3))
 (segment (start 96 84.2) (end 96 81.09) (width 0.2) (layer "B.Cu") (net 3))
 (segment (start 97.2 85.4) (end 96 84.2) (width 0.2) (layer "B.Cu") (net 3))
 (segment (start 101.45 86.21) (end 103.96 86.21) (width 0.2) (layer "F.Cu") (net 14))
 (segment (start 103.96 86.21) (end 106.35 83.82) (width 0.2) (layer "F.Cu") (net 14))
 (segment (start 93.8 86.21) (end 93.65 86.36) (width 0.2) (layer "F.Cu") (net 4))
 (segment (start 98.55 86.21) (end 93.8 86.21) (width 0.2) (layer "F.Cu") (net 4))
 (segment (start 104.3 84.7) (end 103.19 85.81) (width 0.2) (layer "F.Cu") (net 15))
 (segment (start 103.19 85.81) (end 101.45 85.81) (width 0.2) (layer "F.Cu") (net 15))
 (via (at 104.3 84.7) (size 0.8) (drill 0.4) (layers "F.Cu" "B.Cu") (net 15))
 (segment (start 104.3 80.79) (end 106.35 78.74) (width 0.2) (layer "B.Cu") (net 15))
 (segment (start 104.3 84.7) (end 104.3 80.79) (width 0.2) (layer "B.Cu") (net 15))
 (segment (start 106.35 81.65) (end 106.35 81.28) (width 0.2) (layer "F.Cu") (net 16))
 (segment (start 100.9 84.6) (end 103.4 84.6) (width 0.2) (layer "F.Cu") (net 16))
 (segment (start 103.4 84.6) (end 106.35 81.65) (width 0.2) (layer "F.Cu") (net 16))
 (segment (start 100.8 85.16) (end 100.8 84.7) (width 0.2) (layer "F.Cu") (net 16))
 (segment (start 100.8 84.7) (end 100.9 84.6) (width 0.2) (layer "F.Cu") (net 16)))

